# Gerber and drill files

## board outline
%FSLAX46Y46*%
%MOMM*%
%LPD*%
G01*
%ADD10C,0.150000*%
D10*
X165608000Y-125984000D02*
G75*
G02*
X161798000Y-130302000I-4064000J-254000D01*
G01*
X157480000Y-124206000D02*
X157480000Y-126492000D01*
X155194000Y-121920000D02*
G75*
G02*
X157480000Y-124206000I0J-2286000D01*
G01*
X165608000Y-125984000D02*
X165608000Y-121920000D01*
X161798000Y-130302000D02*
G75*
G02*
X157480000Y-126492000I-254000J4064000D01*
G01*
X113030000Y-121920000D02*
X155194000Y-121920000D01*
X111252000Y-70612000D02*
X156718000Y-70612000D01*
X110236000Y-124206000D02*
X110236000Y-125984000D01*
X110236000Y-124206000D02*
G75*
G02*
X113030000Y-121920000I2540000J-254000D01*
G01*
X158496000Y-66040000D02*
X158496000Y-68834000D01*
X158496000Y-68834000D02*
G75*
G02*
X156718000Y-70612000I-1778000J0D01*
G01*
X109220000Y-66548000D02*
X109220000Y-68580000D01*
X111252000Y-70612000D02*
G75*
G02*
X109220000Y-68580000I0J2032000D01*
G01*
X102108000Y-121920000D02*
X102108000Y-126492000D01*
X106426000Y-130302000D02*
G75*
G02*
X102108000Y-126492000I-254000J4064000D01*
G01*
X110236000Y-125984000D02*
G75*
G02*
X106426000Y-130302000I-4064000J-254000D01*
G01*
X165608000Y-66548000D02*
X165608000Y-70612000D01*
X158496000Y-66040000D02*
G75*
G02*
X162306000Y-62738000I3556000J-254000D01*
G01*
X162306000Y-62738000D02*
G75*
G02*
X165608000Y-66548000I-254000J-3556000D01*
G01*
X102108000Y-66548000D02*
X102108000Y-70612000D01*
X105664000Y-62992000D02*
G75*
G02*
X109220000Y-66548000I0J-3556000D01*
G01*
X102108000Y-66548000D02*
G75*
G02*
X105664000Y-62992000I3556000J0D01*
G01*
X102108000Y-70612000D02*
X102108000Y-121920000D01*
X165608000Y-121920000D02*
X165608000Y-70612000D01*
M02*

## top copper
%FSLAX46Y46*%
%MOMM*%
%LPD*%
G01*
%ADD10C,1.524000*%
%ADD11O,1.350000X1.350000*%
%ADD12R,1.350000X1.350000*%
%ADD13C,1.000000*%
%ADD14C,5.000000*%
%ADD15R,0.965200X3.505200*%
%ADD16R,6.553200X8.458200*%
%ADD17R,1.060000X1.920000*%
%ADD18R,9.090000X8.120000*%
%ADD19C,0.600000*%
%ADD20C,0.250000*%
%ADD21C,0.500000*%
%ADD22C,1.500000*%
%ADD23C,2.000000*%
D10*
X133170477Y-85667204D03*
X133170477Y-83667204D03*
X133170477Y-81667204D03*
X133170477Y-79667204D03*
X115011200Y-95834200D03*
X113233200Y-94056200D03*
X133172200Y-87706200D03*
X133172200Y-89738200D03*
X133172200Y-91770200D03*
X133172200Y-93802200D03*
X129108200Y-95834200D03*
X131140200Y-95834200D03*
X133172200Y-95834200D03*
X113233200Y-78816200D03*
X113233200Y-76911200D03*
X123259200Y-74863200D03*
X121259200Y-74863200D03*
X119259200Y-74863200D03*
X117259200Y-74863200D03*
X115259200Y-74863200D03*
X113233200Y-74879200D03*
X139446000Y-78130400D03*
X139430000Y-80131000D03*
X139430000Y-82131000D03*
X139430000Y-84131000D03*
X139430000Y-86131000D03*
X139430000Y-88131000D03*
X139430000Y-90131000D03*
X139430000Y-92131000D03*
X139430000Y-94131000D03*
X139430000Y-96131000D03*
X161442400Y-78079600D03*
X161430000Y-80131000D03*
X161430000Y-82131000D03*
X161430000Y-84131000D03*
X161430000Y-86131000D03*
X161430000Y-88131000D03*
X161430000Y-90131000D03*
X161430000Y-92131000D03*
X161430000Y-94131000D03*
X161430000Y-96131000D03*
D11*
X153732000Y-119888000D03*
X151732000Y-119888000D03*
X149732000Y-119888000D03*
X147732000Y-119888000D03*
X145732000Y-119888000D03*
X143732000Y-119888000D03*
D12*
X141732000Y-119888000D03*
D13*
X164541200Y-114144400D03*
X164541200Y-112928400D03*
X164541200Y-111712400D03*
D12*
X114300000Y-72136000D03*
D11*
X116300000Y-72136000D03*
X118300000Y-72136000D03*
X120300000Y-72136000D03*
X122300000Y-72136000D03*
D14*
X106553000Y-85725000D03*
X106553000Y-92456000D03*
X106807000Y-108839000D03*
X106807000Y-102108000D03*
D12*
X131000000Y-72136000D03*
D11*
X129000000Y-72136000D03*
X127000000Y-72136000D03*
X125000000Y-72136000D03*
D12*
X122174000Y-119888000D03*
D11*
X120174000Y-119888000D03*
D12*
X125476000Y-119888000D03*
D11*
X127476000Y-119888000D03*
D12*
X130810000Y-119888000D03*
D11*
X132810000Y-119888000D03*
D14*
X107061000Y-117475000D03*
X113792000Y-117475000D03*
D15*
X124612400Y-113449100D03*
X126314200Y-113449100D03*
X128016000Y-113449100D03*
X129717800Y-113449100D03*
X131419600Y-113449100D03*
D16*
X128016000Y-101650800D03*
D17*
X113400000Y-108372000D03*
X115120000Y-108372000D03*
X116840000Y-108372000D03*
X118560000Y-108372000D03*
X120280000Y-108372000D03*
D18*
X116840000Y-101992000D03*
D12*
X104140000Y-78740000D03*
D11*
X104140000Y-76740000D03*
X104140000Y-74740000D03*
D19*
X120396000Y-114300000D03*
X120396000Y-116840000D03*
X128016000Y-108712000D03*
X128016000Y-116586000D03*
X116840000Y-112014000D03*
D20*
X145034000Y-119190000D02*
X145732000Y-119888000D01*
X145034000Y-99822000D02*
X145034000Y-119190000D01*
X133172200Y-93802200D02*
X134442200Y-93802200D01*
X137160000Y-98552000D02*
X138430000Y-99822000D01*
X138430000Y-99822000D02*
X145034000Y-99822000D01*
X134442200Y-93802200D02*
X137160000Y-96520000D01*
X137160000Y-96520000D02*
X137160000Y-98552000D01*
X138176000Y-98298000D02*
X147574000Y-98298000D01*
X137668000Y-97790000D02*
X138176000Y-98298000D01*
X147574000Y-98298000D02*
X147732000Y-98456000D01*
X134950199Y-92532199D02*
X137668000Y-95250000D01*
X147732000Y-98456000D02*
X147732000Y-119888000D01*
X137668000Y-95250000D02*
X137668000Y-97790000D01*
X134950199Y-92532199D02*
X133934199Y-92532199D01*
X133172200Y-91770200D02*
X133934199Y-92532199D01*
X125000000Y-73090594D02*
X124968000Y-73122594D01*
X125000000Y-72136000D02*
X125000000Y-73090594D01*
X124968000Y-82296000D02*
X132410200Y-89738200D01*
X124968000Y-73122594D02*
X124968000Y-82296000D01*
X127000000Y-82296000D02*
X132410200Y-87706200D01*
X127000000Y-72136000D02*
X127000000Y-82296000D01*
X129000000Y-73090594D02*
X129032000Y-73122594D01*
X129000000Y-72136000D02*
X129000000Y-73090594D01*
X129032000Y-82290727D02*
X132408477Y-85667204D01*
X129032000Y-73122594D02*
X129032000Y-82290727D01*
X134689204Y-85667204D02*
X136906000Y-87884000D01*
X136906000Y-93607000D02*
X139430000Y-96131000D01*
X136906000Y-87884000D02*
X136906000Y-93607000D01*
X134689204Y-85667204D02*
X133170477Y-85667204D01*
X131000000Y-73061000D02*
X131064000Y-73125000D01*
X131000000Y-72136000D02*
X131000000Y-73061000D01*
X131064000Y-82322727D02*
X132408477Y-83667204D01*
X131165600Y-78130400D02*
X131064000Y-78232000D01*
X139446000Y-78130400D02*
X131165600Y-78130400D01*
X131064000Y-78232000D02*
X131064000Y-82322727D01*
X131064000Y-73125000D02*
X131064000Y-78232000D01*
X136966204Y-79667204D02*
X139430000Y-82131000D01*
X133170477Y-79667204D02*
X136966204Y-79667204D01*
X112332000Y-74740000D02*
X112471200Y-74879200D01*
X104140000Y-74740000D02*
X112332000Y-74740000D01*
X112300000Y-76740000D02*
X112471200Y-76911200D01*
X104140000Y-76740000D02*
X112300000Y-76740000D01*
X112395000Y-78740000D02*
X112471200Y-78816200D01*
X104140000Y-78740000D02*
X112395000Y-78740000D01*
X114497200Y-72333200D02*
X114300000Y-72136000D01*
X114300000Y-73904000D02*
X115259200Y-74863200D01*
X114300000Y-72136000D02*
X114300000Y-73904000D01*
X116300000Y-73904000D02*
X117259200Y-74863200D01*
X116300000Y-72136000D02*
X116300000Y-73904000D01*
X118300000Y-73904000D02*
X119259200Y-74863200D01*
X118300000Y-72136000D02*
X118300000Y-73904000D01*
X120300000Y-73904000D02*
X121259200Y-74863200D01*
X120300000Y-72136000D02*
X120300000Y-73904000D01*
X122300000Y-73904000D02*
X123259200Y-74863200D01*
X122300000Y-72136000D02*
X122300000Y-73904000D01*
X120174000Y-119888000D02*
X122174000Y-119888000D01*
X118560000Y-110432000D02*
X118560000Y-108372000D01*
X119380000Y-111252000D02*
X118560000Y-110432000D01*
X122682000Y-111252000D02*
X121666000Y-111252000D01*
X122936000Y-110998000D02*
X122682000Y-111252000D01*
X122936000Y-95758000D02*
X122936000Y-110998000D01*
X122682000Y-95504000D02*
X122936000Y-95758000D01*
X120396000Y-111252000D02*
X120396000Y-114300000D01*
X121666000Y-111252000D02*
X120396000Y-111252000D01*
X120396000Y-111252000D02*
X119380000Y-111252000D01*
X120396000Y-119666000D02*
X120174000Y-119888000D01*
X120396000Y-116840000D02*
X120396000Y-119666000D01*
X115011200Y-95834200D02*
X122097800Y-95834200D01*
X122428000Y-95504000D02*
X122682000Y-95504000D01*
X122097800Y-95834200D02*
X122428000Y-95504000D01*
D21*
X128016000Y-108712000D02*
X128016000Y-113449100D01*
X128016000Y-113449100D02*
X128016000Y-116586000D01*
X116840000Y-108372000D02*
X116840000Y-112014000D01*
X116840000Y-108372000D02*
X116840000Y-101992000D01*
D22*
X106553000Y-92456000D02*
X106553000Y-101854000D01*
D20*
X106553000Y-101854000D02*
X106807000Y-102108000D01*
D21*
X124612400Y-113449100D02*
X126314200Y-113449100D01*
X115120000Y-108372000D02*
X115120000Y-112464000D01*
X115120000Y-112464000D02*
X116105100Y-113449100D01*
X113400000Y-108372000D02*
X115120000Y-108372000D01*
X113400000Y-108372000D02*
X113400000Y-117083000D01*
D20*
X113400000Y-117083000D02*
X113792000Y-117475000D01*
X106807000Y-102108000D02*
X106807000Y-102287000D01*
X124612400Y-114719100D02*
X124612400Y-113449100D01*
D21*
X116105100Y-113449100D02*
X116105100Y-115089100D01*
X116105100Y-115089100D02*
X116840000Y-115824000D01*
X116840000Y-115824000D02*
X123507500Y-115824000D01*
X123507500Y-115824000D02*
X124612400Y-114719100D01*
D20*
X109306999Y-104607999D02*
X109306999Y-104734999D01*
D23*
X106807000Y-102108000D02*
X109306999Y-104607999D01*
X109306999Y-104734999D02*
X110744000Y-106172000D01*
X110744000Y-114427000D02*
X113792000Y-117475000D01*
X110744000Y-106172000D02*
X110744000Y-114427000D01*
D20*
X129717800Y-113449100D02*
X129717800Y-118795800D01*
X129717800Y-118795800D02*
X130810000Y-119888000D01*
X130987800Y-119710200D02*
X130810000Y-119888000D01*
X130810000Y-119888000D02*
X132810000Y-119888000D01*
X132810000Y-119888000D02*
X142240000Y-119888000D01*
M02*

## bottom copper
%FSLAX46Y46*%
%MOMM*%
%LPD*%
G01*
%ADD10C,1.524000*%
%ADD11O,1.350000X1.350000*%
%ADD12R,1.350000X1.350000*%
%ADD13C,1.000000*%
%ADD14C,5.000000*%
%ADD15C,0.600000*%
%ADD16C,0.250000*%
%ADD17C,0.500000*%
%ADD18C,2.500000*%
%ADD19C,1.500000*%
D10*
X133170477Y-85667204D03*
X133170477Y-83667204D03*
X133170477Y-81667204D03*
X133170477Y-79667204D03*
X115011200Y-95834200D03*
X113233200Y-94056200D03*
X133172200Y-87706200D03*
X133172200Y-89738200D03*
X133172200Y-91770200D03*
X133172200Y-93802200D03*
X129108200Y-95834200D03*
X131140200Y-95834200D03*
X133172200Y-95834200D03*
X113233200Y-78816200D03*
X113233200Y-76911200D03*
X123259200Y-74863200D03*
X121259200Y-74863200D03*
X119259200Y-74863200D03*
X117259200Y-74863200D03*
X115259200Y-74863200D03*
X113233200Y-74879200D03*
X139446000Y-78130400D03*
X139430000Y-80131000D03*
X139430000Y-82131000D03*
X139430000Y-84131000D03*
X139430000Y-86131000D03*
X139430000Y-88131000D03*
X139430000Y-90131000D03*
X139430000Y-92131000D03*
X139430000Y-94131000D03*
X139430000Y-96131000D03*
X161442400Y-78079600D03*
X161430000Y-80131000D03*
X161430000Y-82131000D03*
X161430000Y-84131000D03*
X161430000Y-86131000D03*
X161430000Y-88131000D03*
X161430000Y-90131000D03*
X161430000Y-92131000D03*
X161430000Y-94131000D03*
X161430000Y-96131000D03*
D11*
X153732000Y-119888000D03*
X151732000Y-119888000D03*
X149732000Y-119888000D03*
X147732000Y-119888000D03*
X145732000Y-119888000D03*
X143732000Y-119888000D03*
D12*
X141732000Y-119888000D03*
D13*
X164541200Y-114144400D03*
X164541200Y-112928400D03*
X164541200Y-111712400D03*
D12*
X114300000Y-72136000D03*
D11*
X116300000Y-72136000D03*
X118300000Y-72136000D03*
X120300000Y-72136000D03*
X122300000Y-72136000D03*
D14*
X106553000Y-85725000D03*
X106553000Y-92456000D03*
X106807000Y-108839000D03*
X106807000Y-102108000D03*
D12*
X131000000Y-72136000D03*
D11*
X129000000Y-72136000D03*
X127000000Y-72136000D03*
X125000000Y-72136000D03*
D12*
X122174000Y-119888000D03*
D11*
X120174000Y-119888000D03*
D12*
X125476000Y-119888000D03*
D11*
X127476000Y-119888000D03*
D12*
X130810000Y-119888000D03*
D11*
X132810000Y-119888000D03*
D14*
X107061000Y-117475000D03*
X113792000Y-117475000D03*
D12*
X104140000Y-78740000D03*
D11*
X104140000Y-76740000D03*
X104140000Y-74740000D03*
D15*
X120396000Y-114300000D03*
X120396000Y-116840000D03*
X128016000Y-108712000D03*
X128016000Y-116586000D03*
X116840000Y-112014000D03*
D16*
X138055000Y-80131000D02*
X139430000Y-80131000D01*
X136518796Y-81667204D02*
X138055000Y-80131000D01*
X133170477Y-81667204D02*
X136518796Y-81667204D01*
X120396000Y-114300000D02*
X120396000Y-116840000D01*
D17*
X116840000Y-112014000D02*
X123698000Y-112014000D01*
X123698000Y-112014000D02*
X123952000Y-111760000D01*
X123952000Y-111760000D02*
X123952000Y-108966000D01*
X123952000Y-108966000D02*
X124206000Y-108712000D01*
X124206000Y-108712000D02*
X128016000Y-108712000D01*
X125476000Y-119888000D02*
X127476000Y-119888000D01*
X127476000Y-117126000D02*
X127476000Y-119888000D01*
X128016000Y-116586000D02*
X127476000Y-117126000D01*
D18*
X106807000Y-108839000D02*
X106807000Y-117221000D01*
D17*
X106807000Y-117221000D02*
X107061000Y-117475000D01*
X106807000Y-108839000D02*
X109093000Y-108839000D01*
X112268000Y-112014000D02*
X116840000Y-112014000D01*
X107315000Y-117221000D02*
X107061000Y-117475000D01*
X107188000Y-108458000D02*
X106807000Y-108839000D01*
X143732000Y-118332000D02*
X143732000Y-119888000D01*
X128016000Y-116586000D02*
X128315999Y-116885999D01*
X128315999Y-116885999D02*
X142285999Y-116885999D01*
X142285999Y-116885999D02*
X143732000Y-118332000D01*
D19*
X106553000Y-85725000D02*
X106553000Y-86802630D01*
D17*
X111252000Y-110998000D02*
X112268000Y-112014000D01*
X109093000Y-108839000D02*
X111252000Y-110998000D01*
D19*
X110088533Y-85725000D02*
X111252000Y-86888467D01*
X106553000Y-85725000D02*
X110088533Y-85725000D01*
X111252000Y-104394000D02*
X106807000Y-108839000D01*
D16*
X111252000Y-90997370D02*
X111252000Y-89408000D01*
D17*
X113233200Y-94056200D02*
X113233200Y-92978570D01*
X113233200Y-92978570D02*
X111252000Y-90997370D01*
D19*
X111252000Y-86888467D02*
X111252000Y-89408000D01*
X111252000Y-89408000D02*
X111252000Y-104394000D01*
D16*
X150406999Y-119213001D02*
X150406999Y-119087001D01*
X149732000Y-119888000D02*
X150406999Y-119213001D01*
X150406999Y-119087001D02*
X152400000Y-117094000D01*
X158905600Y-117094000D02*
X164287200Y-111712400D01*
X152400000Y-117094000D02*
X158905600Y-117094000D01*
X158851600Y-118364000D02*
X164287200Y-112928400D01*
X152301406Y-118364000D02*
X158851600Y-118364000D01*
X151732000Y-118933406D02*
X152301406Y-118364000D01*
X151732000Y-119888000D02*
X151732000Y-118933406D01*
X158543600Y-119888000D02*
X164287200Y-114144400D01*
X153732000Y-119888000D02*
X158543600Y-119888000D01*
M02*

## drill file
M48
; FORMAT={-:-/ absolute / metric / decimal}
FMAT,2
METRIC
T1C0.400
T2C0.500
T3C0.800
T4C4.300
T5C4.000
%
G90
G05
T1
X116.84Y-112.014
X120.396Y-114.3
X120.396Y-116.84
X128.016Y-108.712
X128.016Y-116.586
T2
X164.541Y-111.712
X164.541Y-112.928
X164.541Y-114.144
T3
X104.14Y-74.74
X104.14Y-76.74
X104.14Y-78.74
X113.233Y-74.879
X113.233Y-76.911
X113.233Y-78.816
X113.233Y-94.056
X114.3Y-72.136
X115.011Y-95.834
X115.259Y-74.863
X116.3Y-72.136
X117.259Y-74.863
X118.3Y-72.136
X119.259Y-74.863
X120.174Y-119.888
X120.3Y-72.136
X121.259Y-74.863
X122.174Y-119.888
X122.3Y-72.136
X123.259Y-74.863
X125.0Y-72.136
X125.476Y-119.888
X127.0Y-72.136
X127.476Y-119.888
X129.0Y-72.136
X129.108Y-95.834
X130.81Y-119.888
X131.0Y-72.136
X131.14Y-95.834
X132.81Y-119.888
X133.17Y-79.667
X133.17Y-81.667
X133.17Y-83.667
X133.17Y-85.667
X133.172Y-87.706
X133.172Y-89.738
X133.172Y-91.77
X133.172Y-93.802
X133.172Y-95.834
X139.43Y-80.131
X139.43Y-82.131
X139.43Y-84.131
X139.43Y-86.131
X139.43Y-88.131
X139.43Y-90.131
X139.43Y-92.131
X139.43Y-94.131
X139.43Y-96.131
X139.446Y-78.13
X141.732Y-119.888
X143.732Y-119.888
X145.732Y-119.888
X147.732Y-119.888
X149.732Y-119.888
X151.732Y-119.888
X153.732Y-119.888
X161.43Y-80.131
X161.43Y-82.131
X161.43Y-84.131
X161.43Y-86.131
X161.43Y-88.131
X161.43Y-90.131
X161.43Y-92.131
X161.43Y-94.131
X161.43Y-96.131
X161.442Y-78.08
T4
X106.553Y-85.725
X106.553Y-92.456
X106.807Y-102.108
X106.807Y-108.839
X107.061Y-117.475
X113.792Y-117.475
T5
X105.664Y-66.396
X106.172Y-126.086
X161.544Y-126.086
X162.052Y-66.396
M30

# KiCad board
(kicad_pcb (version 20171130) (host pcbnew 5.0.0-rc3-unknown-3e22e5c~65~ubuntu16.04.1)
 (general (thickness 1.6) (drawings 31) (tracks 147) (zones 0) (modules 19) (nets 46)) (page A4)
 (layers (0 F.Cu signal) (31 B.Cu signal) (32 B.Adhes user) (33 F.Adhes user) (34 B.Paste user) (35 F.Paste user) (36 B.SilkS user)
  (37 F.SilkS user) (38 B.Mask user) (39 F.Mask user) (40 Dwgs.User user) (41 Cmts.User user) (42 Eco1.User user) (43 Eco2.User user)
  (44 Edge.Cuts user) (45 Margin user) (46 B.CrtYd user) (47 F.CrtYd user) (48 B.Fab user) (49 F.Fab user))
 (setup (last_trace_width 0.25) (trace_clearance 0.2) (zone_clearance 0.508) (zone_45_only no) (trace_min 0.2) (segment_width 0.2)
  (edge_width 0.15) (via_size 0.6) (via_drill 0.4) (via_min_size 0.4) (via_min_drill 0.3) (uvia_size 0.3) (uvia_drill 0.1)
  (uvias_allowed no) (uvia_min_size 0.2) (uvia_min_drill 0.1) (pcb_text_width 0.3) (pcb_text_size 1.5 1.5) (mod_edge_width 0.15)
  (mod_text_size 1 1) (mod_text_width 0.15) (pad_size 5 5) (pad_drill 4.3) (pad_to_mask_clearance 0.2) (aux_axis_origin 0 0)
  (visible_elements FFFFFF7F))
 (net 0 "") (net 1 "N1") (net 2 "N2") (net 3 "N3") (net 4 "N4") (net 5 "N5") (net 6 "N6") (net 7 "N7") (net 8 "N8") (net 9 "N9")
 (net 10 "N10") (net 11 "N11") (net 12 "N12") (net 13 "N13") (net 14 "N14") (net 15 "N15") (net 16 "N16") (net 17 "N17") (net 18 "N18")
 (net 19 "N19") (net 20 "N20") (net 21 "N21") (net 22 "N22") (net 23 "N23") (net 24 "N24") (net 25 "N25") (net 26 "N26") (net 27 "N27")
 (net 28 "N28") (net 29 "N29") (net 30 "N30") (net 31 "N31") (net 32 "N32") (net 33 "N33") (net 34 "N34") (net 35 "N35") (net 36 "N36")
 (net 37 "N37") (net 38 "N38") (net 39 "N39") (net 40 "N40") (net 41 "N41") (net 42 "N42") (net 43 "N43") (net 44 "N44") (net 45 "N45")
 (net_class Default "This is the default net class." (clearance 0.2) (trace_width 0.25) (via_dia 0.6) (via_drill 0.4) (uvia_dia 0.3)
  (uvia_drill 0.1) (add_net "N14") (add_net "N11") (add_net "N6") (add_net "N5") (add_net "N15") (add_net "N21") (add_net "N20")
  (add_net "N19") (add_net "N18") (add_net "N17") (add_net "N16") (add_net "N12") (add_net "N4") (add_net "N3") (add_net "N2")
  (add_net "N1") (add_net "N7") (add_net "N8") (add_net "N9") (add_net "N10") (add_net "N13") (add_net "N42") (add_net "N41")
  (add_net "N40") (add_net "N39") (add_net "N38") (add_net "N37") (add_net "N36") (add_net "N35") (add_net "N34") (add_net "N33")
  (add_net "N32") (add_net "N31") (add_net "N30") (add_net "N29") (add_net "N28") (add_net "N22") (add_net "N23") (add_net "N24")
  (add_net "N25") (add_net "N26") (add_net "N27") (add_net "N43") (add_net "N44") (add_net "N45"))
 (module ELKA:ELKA (layer F.Cu) (at 122.428 85.852)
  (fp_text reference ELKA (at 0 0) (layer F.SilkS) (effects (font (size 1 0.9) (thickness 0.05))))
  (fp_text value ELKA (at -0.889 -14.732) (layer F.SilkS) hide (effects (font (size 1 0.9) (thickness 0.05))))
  (pad D thru_hole circle (at 10.742477 -0.184796 270) (size 1.524 1.524) (drill 0.8) (layers *.Cu *.Mask B.SilkS) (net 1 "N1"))
  (pad C thru_hole circle (at 10.742477 -2.184796 270) (size 1.524 1.524) (drill 0.8) (layers *.Cu *.Mask B.SilkS) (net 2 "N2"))
  (pad B thru_hole circle (at 10.742477 -4.184796 270) (size 1.524 1.524) (drill 0.8) (layers *.Cu *.Mask B.SilkS) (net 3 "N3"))
  (pad A thru_hole circle (at 10.742477 -6.184796 270) (size 1.524 1.524) (drill 0.8) (layers *.Cu *.Mask B.SilkS) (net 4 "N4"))
  (pad 12 thru_hole circle (at -7.4168 9.9822 270) (size 1.524 1.524) (drill 0.8) (layers *.Cu *.Mask B.SilkS) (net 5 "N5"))
  (pad 11 thru_hole circle (at -9.1948 8.2042 270) (size 1.524 1.524) (drill 0.8) (layers *.Cu *.Mask B.SilkS) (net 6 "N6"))
  (pad E thru_hole circle (at 10.7442 1.8542 270) (size 1.524 1.524) (drill 0.8) (layers *.Cu *.Mask B.SilkS) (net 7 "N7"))
  (pad F thru_hole circle (at 10.7442 3.8862 270) (size 1.524 1.524) (drill 0.8) (layers *.Cu *.Mask B.SilkS) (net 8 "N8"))
  (pad G thru_hole circle (at 10.7442 5.9182 270) (size 1.524 1.524) (drill 0.8) (layers *.Cu *.Mask B.SilkS) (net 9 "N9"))
  (pad H thru_hole circle (at 10.7442 7.9502 270) (size 1.524 1.524) (drill 0.8) (layers *.Cu *.Mask B.SilkS) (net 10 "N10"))
  (pad 10 thru_hole circle (at 6.6802 9.9822 270) (size 1.524 1.524) (drill 0.8) (layers *.Cu *.Mask B.SilkS) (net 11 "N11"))
  (pad 9 thru_hole circle (at 8.7122 9.9822 270) (size 1.524 1.524) (drill 0.8) (layers *.Cu *.Mask B.SilkS) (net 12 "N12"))
  (pad I thru_hole circle (at 10.7442 9.9822 270) (size 1.524 1.524) (drill 0.8) (layers *.Cu *.Mask B.SilkS) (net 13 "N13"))
  (pad 1 thru_hole circle (at -9.1948 -7.0358 270) (size 1.524 1.524) (drill 0.8) (layers *.Cu *.Mask B.SilkS) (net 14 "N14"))
  (pad 2 thru_hole circle (at -9.1948 -8.9408 270) (size 1.524 1.524) (drill 0.8) (layers *.Cu *.Mask B.SilkS) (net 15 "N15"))
  (pad 8 thru_hole circle (at 0.8312 -10.9888 270) (size 1.524 1.524) (drill 0.8) (layers *.Cu *.Mask B.SilkS) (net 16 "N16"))
  (pad 7 thru_hole circle (at -1.1688 -10.9888 270) (size 1.524 1.524) (drill 0.8) (layers *.Cu *.Mask B.SilkS) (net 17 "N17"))
  (pad 6 thru_hole circle (at -3.1688 -10.9888 270) (size 1.524 1.524) (drill 0.8) (layers *.Cu *.Mask B.SilkS) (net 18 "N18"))
  (pad 5 thru_hole circle (at -5.1688 -10.9888 270) (size 1.524 1.524) (drill 0.8) (layers *.Cu *.Mask B.SilkS) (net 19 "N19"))
  (pad 4 thru_hole circle (at -7.1688 -10.9888 270) (size 1.524 1.524) (drill 0.8) (layers *.Cu *.Mask B.SilkS) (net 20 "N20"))
  (pad 3 thru_hole circle (at -9.1948 -10.9728 270) (size 1.524 1.524) (drill 0.8) (layers *.Cu *.Mask B.SilkS) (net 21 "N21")))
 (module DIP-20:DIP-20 (layer F.Cu) (at 138.176 104.14)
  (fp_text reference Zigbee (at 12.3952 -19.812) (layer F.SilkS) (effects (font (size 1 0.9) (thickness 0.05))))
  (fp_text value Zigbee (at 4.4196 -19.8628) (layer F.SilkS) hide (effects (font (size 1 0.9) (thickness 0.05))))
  (pad 1 thru_hole circle (at 1.27 -26.0096) (size 1.524 1.524) (drill 0.8) (layers *.Cu *.Mask F.SilkS) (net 2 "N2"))
  (pad 2 thru_hole circle (at 1.254 -24.009) (size 1.524 1.524) (drill 0.8) (layers *.Cu *.Mask F.SilkS) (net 3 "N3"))
  (pad 3 thru_hole circle (at 1.254 -22.009) (size 1.524 1.524) (drill 0.8) (layers *.Cu *.Mask F.SilkS) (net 4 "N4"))
  (pad 4 thru_hole circle (at 1.254 -20.009) (size 1.524 1.524) (drill 0.8) (layers *.Cu *.Mask F.SilkS) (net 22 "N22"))
  (pad 5 thru_hole circle (at 1.254 -18.009) (size 1.524 1.524) (drill 0.8) (layers *.Cu *.Mask F.SilkS) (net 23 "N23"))
  (pad 6 thru_hole circle (at 1.254 -16.009) (size 1.524 1.524) (drill 0.8) (layers *.Cu *.Mask F.SilkS) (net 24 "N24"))
  (pad 7 thru_hole circle (at 1.254 -14.009) (size 1.524 1.524) (drill 0.8) (layers *.Cu *.Mask F.SilkS) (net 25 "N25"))
  (pad 8 thru_hole circle (at 1.254 -12.009) (size 1.524 1.524) (drill 0.8) (layers *.Cu *.Mask F.SilkS) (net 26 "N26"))
  (pad 9 thru_hole circle (at 1.254 -10.009) (size 1.524 1.524) (drill 0.8) (layers *.Cu *.Mask F.SilkS) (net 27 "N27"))
  (pad 10 thru_hole circle (at 1.254 -8.009) (size 1.524 1.524) (drill 0.8) (layers *.Cu *.Mask F.SilkS) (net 1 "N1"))
  (pad 20 thru_hole circle (at 23.2664 -26.0604) (size 1.524 1.524) (drill 0.8) (layers *.Cu *.Mask F.SilkS) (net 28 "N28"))
  (pad 19 thru_hole circle (at 23.254 -24.009) (size 1.524 1.524) (drill 0.8) (layers *.Cu *.Mask F.SilkS) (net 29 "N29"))
  (pad 18 thru_hole circle (at 23.254 -22.009) (size 1.524 1.524) (drill 0.8) (layers *.Cu *.Mask F.SilkS) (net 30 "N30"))
  (pad 17 thru_hole circle (at 23.254 -20.009) (size 1.524 1.524) (drill 0.8) (layers *.Cu *.Mask F.SilkS) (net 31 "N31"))
  (pad 16 thru_hole circle (at 23.254 -18.009) (size 1.524 1.524) (drill 0.8) (layers *.Cu *.Mask F.SilkS) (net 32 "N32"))
  (pad 15 thru_hole circle (at 23.254 -16.009) (size 1.524 1.524) (drill 0.8) (layers *.Cu *.Mask F.SilkS) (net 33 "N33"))
  (pad 14 thru_hole circle (at 23.254 -14.009) (size 1.524 1.524) (drill 0.8) (layers *.Cu *.Mask F.SilkS) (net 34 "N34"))
  (pad 13 thru_hole circle (at 23.254 -12.009) (size 1.524 1.524) (drill 0.8) (layers *.Cu *.Mask F.SilkS) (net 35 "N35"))
  (pad 12 thru_hole circle (at 23.254 -10.009) (size 1.524 1.524) (drill 0.8) (layers *.Cu *.Mask F.SilkS) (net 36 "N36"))
  (pad 11 thru_hole circle (at 23.254 -8.009) (size 1.524 1.524) (drill 0.8) (layers *.Cu *.Mask F.SilkS) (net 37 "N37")))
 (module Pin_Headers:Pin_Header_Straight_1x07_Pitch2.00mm (layer F.Cu) (at 141.732 119.888 90)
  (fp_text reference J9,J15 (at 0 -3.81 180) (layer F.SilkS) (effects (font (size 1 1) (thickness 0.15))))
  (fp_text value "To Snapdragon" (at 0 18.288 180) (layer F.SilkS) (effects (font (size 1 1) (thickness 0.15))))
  (pad 5 thru_hole oval (at 0 12 90) (size 1.35 1.35) (drill 0.8) (layers *.Cu *.Mask) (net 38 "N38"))
  (pad 4 thru_hole oval (at 0 10 90) (size 1.35 1.35) (drill 0.8) (layers *.Cu *.Mask) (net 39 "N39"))
  (pad 3 thru_hole oval (at 0 8 90) (size 1.35 1.35) (drill 0.8) (layers *.Cu *.Mask) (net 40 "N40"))
  (pad 6 thru_hole oval (at 0 6 90) (size 1.35 1.35) (drill 0.8) (layers *.Cu *.Mask) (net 9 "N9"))
  (pad 7 thru_hole oval (at 0 4 90) (size 1.35 1.35) (drill 0.8) (layers *.Cu *.Mask) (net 10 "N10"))
  (pad 2 thru_hole oval (at 0 2 90) (size 1.35 1.35) (drill 0.8) (layers *.Cu *.Mask) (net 6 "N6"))
  (pad 1 thru_hole rect (at 0 0 90) (size 1.35 1.35) (drill 0.8) (layers *.Cu *.Mask) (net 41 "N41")))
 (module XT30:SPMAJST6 (layer F.Cu) (at 163.83 113.792 270)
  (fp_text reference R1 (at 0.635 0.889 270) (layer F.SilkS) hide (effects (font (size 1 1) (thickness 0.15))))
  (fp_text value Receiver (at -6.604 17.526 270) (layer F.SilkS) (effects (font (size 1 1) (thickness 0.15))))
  (pad 3 thru_hole circle (at 0.3524 -0.7112 270) (size 1 1) (drill 0.5) (layers *.Cu *.Mask) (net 38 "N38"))
  (pad 2 thru_hole circle (at -0.8636 -0.7112 270) (size 1 1) (drill 0.5) (layers *.Cu *.Mask) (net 39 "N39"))
  (pad 1 thru_hole circle (at -2.0796 -0.7112 270) (size 1 1) (drill 0.5) (layers *.Cu *.Mask) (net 40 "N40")))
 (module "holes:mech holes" (layer F.Cu) (at 162.052 129.286)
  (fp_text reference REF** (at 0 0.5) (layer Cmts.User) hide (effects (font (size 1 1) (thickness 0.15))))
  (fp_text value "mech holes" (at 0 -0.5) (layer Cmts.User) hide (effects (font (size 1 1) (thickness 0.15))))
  (pad "" np_thru_hole circle (at -0.508 -3.2004) (size 4 4) (drill 4) (layers *.Cu *.Mask)))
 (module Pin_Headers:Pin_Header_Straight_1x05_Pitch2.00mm (layer F.Cu) (at 114.3 72.136 90)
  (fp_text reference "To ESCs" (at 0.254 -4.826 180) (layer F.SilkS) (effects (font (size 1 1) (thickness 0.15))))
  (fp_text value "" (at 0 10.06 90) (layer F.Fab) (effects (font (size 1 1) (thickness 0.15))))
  (pad 1 thru_hole rect (at 0 0 90) (size 1.35 1.35) (drill 0.8) (layers *.Cu *.Mask) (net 20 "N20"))
  (pad 2 thru_hole oval (at 0 2 90) (size 1.35 1.35) (drill 0.8) (layers *.Cu *.Mask) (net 19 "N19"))
  (pad 3 thru_hole oval (at 0 4 90) (size 1.35 1.35) (drill 0.8) (layers *.Cu *.Mask) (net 18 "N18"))
  (pad 4 thru_hole oval (at 0 6 90) (size 1.35 1.35) (drill 0.8) (layers *.Cu *.Mask) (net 17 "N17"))
  (pad 5 thru_hole oval (at 0 8 90) (size 1.35 1.35) (drill 0.8) (layers *.Cu *.Mask) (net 16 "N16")))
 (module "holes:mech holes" (layer F.Cu) (at 106.172 69.596)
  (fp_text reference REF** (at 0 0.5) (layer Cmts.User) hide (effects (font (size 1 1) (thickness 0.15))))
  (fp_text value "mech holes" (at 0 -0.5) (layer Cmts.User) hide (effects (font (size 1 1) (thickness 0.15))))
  (pad "" np_thru_hole circle (at -0.508 -3.2004) (size 4 4) (drill 4) (layers *.Cu *.Mask)))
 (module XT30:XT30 (layer F.Cu) (at 112.522 87.122 270)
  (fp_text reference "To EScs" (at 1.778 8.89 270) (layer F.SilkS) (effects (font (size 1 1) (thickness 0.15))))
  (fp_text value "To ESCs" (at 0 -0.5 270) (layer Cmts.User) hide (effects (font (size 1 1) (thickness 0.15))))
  (pad 1 thru_hole circle (at -1.397 5.969 270) (size 5 5) (drill 4.3) (layers *.Cu *.Mask) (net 6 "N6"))
  (pad 2 thru_hole circle (at 5.334 5.969 270) (size 5 5) (drill 4.3) (layers *.Cu *.Mask) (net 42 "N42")))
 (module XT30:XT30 (layer F.Cu) (at 100.838 107.442 90)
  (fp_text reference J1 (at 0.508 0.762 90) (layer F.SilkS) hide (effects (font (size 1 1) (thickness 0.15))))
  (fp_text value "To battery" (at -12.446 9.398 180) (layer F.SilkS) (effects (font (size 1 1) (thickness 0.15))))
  (pad 1 thru_hole circle (at -1.397 5.969 90) (size 5 5) (drill 4.3) (layers *.Cu *.Mask) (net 6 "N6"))
  (pad 2 thru_hole circle (at 5.334 5.969 90) (size 5 5) (drill 4.3) (layers *.Cu *.Mask) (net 42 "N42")))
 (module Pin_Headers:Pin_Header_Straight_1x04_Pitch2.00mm (layer F.Cu) (at 131 72.136 270)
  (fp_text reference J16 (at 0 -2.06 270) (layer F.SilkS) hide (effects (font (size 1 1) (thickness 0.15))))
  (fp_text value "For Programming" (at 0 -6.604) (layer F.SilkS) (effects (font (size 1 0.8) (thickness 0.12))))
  (pad 1 thru_hole rect (at 0 0 270) (size 1.35 1.35) (drill 0.8) (layers *.Cu *.Mask) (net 2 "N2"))
  (pad 2 thru_hole oval (at 0 2 270) (size 1.35 1.35) (drill 0.8) (layers *.Cu *.Mask) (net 1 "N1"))
  (pad 3 thru_hole oval (at 0 4 270) (size 1.35 1.35) (drill 0.8) (layers *.Cu *.Mask) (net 7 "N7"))
  (pad 4 thru_hole oval (at 0 6 270) (size 1.35 1.35) (drill 0.8) (layers *.Cu *.Mask) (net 8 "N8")))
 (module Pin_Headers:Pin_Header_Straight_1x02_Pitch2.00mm (layer F.Cu) (at 122.174 119.888 270)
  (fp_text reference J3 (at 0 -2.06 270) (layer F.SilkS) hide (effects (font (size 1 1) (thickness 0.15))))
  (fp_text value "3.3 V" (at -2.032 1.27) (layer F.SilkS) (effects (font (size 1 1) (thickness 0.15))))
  (pad 1 thru_hole rect (at 0 0 270) (size 1.35 1.35) (drill 0.8) (layers *.Cu *.Mask) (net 5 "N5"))
  (pad 2 thru_hole oval (at 0 2 270) (size 1.35 1.35) (drill 0.8) (layers *.Cu *.Mask) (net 5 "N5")))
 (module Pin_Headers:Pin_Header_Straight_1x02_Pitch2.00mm (layer F.Cu) (at 125.476 119.888 90)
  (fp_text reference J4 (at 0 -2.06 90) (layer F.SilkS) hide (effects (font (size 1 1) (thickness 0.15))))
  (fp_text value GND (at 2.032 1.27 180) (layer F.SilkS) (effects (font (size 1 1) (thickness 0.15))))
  (pad 1 thru_hole rect (at 0 0 90) (size 1.35 1.35) (drill 0.8) (layers *.Cu *.Mask) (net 6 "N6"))
  (pad 2 thru_hole oval (at 0 2 90) (size 1.35 1.35) (drill 0.8) (layers *.Cu *.Mask) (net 6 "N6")))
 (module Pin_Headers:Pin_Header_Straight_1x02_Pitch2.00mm (layer F.Cu) (at 130.81 119.888 90)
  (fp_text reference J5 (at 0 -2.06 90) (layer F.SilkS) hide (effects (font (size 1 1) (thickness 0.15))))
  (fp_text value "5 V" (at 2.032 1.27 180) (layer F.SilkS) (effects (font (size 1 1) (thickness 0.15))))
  (pad 1 thru_hole rect (at 0 0 90) (size 1.35 1.35) (drill 0.8) (layers *.Cu *.Mask) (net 41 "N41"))
  (pad 2 thru_hole oval (at 0 2 90) (size 1.35 1.35) (drill 0.8) (layers *.Cu *.Mask) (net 41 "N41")))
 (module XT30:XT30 (layer F.Cu) (at 108.458 111.506)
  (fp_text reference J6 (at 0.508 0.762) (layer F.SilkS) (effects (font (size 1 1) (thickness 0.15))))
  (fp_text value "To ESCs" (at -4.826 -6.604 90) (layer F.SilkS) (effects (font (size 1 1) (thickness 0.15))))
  (pad 1 thru_hole circle (at -1.397 5.969) (size 5 5) (drill 4.3) (layers *.Cu *.Mask) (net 6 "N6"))
  (pad 2 thru_hole circle (at 5.334 5.969) (size 5 5) (drill 4.3) (layers *.Cu *.Mask) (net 42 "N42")))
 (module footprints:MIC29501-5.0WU (layer F.Cu) (at 128.016 104.394)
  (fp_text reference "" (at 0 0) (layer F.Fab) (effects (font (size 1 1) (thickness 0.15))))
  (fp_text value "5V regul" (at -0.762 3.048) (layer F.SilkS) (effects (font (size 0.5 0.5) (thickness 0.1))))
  (pad 1 smd rect (at -3.4036 9.0551) (size 0.9652 3.5052) (layers F.Cu F.Paste F.Mask) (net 42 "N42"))
  (pad 2 smd rect (at -1.7018 9.0551) (size 0.9652 3.5052) (layers F.Cu F.Paste F.Mask) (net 42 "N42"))
  (pad 3 smd rect (at 0 9.0551) (size 0.9652 3.5052) (layers F.Cu F.Paste F.Mask) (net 6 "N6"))
  (pad 4 smd rect (at 1.7018 9.0551) (size 0.9652 3.5052) (layers F.Cu F.Paste F.Mask) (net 41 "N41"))
  (pad 5 smd rect (at 3.4036 9.0551) (size 0.9652 3.5052) (layers F.Cu F.Paste F.Mask) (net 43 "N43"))
  (pad 6 smd rect (at 0 -2.7432) (size 6.5532 8.4582) (layers F.Cu F.Paste F.Mask) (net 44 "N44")))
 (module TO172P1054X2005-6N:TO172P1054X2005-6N (layer F.Cu) (at 116.84 103.632)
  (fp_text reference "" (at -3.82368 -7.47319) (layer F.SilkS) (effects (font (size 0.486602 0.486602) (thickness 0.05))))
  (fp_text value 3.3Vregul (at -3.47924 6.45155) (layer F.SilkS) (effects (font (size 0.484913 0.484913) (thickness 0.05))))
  (pad 1 smd rect (at -3.44 4.74 90) (size 1.92 1.06) (layers F.Cu F.Paste F.Mask) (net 42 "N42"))
  (pad 2 smd rect (at -1.72 4.74 90) (size 1.92 1.06) (layers F.Cu F.Paste F.Mask) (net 42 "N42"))
  (pad 3 smd rect (at 0 4.74 90) (size 1.92 1.06) (layers F.Cu F.Paste F.Mask) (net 6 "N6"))
  (pad 4 smd rect (at 1.72 4.74 90) (size 1.92 1.06) (layers F.Cu F.Paste F.Mask) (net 5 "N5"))
  (pad 5 smd rect (at 3.44 4.74 90) (size 1.92 1.06) (layers F.Cu F.Paste F.Mask) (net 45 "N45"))
  (pad 6 smd rect (at 0 -1.64 90) (size 8.12 9.09) (layers F.Cu F.Paste F.Mask) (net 6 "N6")))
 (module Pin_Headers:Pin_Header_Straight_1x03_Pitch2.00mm (layer F.Cu) (at 104.14 78.74 180)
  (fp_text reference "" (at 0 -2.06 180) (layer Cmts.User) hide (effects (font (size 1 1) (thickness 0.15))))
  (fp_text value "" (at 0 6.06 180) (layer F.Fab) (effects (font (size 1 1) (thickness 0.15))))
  (pad 1 thru_hole rect (at 0 0 180) (size 1.35 1.35) (drill 0.8) (layers *.Cu *.Mask) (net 14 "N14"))
  (pad 2 thru_hole oval (at 0 2 180) (size 1.35 1.35) (drill 0.8) (layers *.Cu *.Mask) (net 15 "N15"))
  (pad 3 thru_hole oval (at 0 4 180) (size 1.35 1.35) (drill 0.8) (layers *.Cu *.Mask) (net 21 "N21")))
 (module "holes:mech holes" (layer F.Cu) (at 162.56 69.596)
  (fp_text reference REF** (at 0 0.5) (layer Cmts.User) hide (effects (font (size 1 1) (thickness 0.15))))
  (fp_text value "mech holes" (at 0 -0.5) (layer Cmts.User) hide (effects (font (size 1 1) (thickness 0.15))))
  (pad "" np_thru_hole circle (at -0.508 -3.2004) (size 4 4) (drill 4) (layers *.Cu *.Mask)))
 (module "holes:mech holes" (layer F.Cu) (at 106.68 129.286)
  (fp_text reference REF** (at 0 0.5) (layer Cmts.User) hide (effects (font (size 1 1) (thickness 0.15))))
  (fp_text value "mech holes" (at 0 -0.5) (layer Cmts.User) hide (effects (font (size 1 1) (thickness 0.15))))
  (pad "" np_thru_hole circle (at -0.508 -3.2004) (size 4 4) (drill 4) (layers *.Cu *.Mask)))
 (gr_arc (start 161.544 126.238) (end 165.608 125.984) (angle 90) (layer Edge.Cuts) (width 0.15))
 (gr_line (start 157.48 124.206) (end 157.48 126.492) (angle 90) (layer Edge.Cuts) (width 0.15))
 (gr_arc (start 155.194 124.206) (end 155.194 121.92) (angle 90) (layer Edge.Cuts) (width 0.15))
 (gr_line (start 165.608 125.984) (end 165.608 121.92) (angle 90) (layer Edge.Cuts) (width 0.15))
 (gr_arc (start 161.544 126.238) (end 161.798 130.302) (angle 90) (layer Edge.Cuts) (width 0.15))
 (gr_line (start 113.03 121.92) (end 155.194 121.92) (angle 90) (layer Edge.Cuts) (width 0.15))
 (gr_line (start 111.252 70.612) (end 156.718 70.612) (angle 90) (layer Edge.Cuts) (width 0.15))
 (gr_line (start 110.236 124.206) (end 110.236 125.984) (angle 90) (layer Edge.Cuts) (width 0.15))
 (gr_arc (start 112.776 124.46) (end 110.236 124.206) (angle 90) (layer Edge.Cuts) (width 0.15))
 (gr_line (start 158.496 66.04) (end 158.496 68.834) (angle 90) (layer Edge.Cuts) (width 0.15))
 (gr_arc (start 156.718 68.834) (end 158.496 68.834) (angle 90) (layer Edge.Cuts) (width 0.15))
 (gr_line (start 109.22 66.548) (end 109.22 68.58) (angle 90) (layer Edge.Cuts) (width 0.15))
 (gr_arc (start 111.252 68.58) (end 111.252 70.612) (angle 90) (layer Edge.Cuts) (width 0.15))
 (gr_line (start 102.108 121.92) (end 102.108 126.492) (angle 90) (layer Edge.Cuts) (width 0.15))
 (gr_arc (start 106.172 126.238) (end 106.426 130.302) (angle 90) (layer Edge.Cuts) (width 0.15))
 (gr_arc (start 106.172 126.238) (end 110.236 125.984) (angle 90) (layer Edge.Cuts) (width 0.15))
 (gr_line (start 165.608 66.548) (end 165.608 70.612) (angle 90) (layer Edge.Cuts) (width 0.15))
 (gr_arc (start 162.052 66.294) (end 158.496 66.04) (angle 90) (layer Edge.Cuts) (width 0.15))
 (gr_arc (start 162.052 66.294) (end 162.306 62.738) (angle 90) (layer Edge.Cuts) (width 0.15))
 (gr_line (start 102.108 66.548) (end 102.108 70.612) (angle 90) (layer Edge.Cuts) (width 0.15))
 (gr_arc (start 105.664 66.548) (end 105.664 62.992) (angle 90) (layer Edge.Cuts) (width 0.15))
 (gr_arc (start 105.664 66.548) (end 102.108 66.548) (angle 90) (layer Edge.Cuts) (width 0.15))
 (gr_line (start 102.108 70.612) (end 102.108 121.92) (angle 90) (layer Edge.Cuts) (width 0.15))
 (gr_line (start 165.608 121.92) (end 165.608 70.612) (angle 90) (layer Edge.Cuts) (width 0.15))
 (segment (start 145.034 119.19) (end 145.732 119.888) (width 0.25) (layer F.Cu) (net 10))
 (segment (start 145.034 99.822) (end 145.034 119.19) (width 0.25) (layer F.Cu) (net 10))
 (segment (start 133.1722 93.8022) (end 134.4422 93.8022) (width 0.25) (layer F.Cu) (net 10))
 (segment (start 137.16 98.552) (end 138.43 99.822) (width 0.25) (layer F.Cu) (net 10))
 (segment (start 138.43 99.822) (end 145.034 99.822) (width 0.25) (layer F.Cu) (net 10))
 (segment (start 134.4422 93.8022) (end 137.16 96.52) (width 0.25) (layer F.Cu) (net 10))
 (segment (start 137.16 96.52) (end 137.16 98.552) (width 0.25) (layer F.Cu) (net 10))
 (segment (start 138.176 98.298) (end 147.574 98.298) (width 0.25) (layer F.Cu) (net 9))
 (segment (start 137.668 97.79) (end 138.176 98.298) (width 0.25) (layer F.Cu) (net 9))
 (segment (start 147.574 98.298) (end 147.732 98.456) (width 0.25) (layer F.Cu) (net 9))
 (segment (start 134.950199 92.532199) (end 137.668 95.25) (width 0.25) (layer F.Cu) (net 9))
 (segment (start 147.732 98.456) (end 147.732 119.888) (width 0.25) (layer F.Cu) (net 9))
 (segment (start 137.668 95.25) (end 137.668 97.79) (width 0.25) (layer F.Cu) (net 9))
 (segment (start 134.950199 92.532199) (end 133.934199 92.532199) (width 0.25) (layer F.Cu) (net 9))
 (segment (start 133.1722 91.7702) (end 133.934199 92.532199) (width 0.25) (layer F.Cu) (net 9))
 (segment (start 125 73.090594) (end 124.968 73.122594) (width 0.25) (layer F.Cu) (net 8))
 (segment (start 125 72.136) (end 125 73.090594) (width 0.25) (layer F.Cu) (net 8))
 (segment (start 124.968 82.296) (end 132.4102 89.7382) (width 0.25) (layer F.Cu) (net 8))
 (segment (start 124.968 73.122594) (end 124.968 82.296) (width 0.25) (layer F.Cu) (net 8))
 (segment (start 127 82.296) (end 132.4102 87.7062) (width 0.25) (layer F.Cu) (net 7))
 (segment (start 127 72.136) (end 127 82.296) (width 0.25) (layer F.Cu) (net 7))
 (segment (start 129 73.090594) (end 129.032 73.122594) (width 0.25) (layer F.Cu) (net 1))
 (segment (start 129 72.136) (end 129 73.090594) (width 0.25) (layer F.Cu) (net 1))
 (segment (start 129.032 82.290727) (end 132.408477 85.667204) (width 0.25) (layer F.Cu) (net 1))
 (segment (start 129.032 73.122594) (end 129.032 82.290727) (width 0.25) (layer F.Cu) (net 1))
 (segment (start 134.689204 85.667204) (end 136.906 87.884) (width 0.25) (layer F.Cu) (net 1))
 (segment (start 136.906 93.607) (end 139.43 96.131) (width 0.25) (layer F.Cu) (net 1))
 (segment (start 136.906 87.884) (end 136.906 93.607) (width 0.25) (layer F.Cu) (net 1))
 (segment (start 134.689204 85.667204) (end 133.170477 85.667204) (width 0.25) (layer F.Cu) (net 1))
 (segment (start 131 73.061) (end 131.064 73.125) (width 0.25) (layer F.Cu) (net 2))
 (segment (start 131 72.136) (end 131 73.061) (width 0.25) (layer F.Cu) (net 2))
 (segment (start 131.064 82.322727) (end 132.408477 83.667204) (width 0.25) (layer F.Cu) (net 2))
 (segment (start 131.1656 78.1304) (end 131.064 78.232) (width 0.25) (layer F.Cu) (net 2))
 (segment (start 139.446 78.1304) (end 131.1656 78.1304) (width 0.25) (layer F.Cu) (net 2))
 (segment (start 131.064 78.232) (end 131.064 82.322727) (width 0.25) (layer F.Cu) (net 2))
 (segment (start 131.064 73.125) (end 131.064 78.232) (width 0.25) (layer F.Cu) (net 2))
 (segment (start 138.055 80.131) (end 139.43 80.131) (width 0.25) (layer B.Cu) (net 3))
 (segment (start 136.518796 81.667204) (end 138.055 80.131) (width 0.25) (layer B.Cu) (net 3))
 (segment (start 133.170477 81.667204) (end 136.518796 81.667204) (width 0.25) (layer B.Cu) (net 3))
 (segment (start 136.966204 79.667204) (end 139.43 82.131) (width 0.25) (layer F.Cu) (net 4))
 (segment (start 133.170477 79.667204) (end 136.966204 79.667204) (width 0.25) (layer F.Cu) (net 4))
 (segment (start 112.332 74.74) (end 112.4712 74.8792) (width 0.25) (layer F.Cu) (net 21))
 (segment (start 104.14 74.74) (end 112.332 74.74) (width 0.25) (layer F.Cu) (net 21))
 (segment (start 112.3 76.74) (end 112.4712 76.9112) (width 0.25) (layer F.Cu) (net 15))
 (segment (start 104.14 76.74) (end 112.3 76.74) (width 0.25) (layer F.Cu) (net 15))
 (segment (start 112.395 78.74) (end 112.4712 78.8162) (width 0.25) (layer F.Cu) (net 14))
 (segment (start 104.14 78.74) (end 112.395 78.74) (width 0.25) (layer F.Cu) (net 14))
 (segment (start 114.4972 72.3332) (end 114.3 72.136) (width 0.25) (layer F.Cu) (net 20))
 (segment (start 114.3 73.904) (end 115.2592 74.8632) (width 0.25) (layer F.Cu) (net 20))
 (segment (start 114.3 72.136) (end 114.3 73.904) (width 0.25) (layer F.Cu) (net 20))
 (segment (start 116.3 73.904) (end 117.2592 74.8632) (width 0.25) (layer F.Cu) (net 19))
 (segment (start 116.3 72.136) (end 116.3 73.904) (width 0.25) (layer F.Cu) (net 19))
 (segment (start 118.3 73.904) (end 119.2592 74.8632) (width 0.25) (layer F.Cu) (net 18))
 (segment (start 118.3 72.136) (end 118.3 73.904) (width 0.25) (layer F.Cu) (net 18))
 (segment (start 120.3 73.904) (end 121.2592 74.8632) (width 0.25) (layer F.Cu) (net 17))
 (segment (start 120.3 72.136) (end 120.3 73.904) (width 0.25) (layer F.Cu) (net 17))
 (segment (start 122.3 73.904) (end 123.2592 74.8632) (width 0.25) (layer F.Cu) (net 16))
 (segment (start 122.3 72.136) (end 122.3 73.904) (width 0.25) (layer F.Cu) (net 16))
 (segment (start 120.174 119.888) (end 122.174 119.888) (width 0.25) (layer F.Cu) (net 5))
 (segment (start 118.56 110.432) (end 118.56 108.372) (width 0.25) (layer F.Cu) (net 5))
 (segment (start 119.38 111.252) (end 118.56 110.432) (width 0.25) (layer F.Cu) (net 5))
 (segment (start 122.682 111.252) (end 121.666 111.252) (width 0.25) (layer F.Cu) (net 5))
 (segment (start 122.936 110.998) (end 122.682 111.252) (width 0.25) (layer F.Cu) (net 5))
 (segment (start 122.936 95.758) (end 122.936 110.998) (width 0.25) (layer F.Cu) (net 5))
 (segment (start 122.682 95.504) (end 122.936 95.758) (width 0.25) (layer F.Cu) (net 5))
 (segment (start 120.396 111.252) (end 120.396 114.3) (width 0.25) (layer F.Cu) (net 5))
 (via (at 120.396 114.3) (size 0.6) (drill 0.4) (layers F.Cu B.Cu) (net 5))
 (segment (start 121.666 111.252) (end 120.396 111.252) (width 0.25) (layer F.Cu) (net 5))
 (segment (start 120.396 111.252) (end 119.38 111.252) (width 0.25) (layer F.Cu) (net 5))
 (via (at 120.396 116.84) (size 0.6) (drill 0.4) (layers F.Cu B.Cu) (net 5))
 (segment (start 120.396 114.3) (end 120.396 116.84) (width 0.25) (layer B.Cu) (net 5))
 (segment (start 120.396 119.666) (end 120.174 119.888) (width 0.25) (layer F.Cu) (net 5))
 (segment (start 120.396 116.84) (end 120.396 119.666) (width 0.25) (layer F.Cu) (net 5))
 (segment (start 115.0112 95.8342) (end 122.0978 95.8342) (width 0.25) (layer F.Cu) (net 5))
 (segment (start 122.428 95.504) (end 122.682 95.504) (width 0.25) (layer F.Cu) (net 5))
 (segment (start 122.0978 95.8342) (end 122.428 95.504) (width 0.25) (layer F.Cu) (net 5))
 (segment (start 116.84 112.014) (end 123.698 112.014) (width 0.5) (layer B.Cu) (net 6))
 (segment (start 123.698 112.014) (end 123.952 111.76) (width 0.5) (layer B.Cu) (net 6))
 (segment (start 123.952 111.76) (end 123.952 108.966) (width 0.5) (layer B.Cu) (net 6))
 (segment (start 123.952 108.966) (end 124.206 108.712) (width 0.5) (layer B.Cu) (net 6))
 (segment (start 124.206 108.712) (end 128.016 108.712) (width 0.5) (layer B.Cu) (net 6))
 (via (at 128.016 108.712) (size 0.6) (drill 0.4) (layers F.Cu B.Cu) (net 6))
 (segment (start 128.016 108.712) (end 128.016 113.4491) (width 0.5) (layer F.Cu) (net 6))
 (segment (start 125.476 119.888) (end 127.476 119.888) (width 0.5) (layer B.Cu) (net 6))
 (segment (start 128.016 113.4491) (end 128.016 116.586) (width 0.5) (layer F.Cu) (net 6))
 (via (at 128.016 116.586) (size 0.6) (drill 0.4) (layers F.Cu B.Cu) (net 6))
 (segment (start 127.476 117.126) (end 127.476 119.888) (width 0.5) (layer B.Cu) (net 6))
 (segment (start 128.016 116.586) (end 127.476 117.126) (width 0.5) (layer B.Cu) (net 6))
 (segment (start 106.807 108.839) (end 106.807 117.221) (width 2.5) (layer B.Cu) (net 6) (status 10))
 (segment (start 106.807 117.221) (end 107.061 117.475) (width 0.5) (layer B.Cu) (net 6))
 (segment (start 116.84 108.372) (end 116.84 112.014) (width 0.5) (layer F.Cu) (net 6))
 (via (at 116.84 112.014) (size 0.6) (drill 0.4) (layers F.Cu B.Cu) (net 6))
 (segment (start 106.807 108.839) (end 109.093 108.839) (width 0.5) (layer B.Cu) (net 6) (status 10))
 (segment (start 112.268 112.014) (end 116.84 112.014) (width 0.5) (layer B.Cu) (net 6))
 (segment (start 107.315 117.221) (end 107.061 117.475) (width 0.5) (layer B.Cu) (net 6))
 (segment (start 107.188 108.458) (end 106.807 108.839) (width 0.5) (layer B.Cu) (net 6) (status 30))
 (segment (start 116.84 108.372) (end 116.84 101.992) (width 0.5) (layer F.Cu) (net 6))
 (segment (start 143.732 118.332) (end 143.732 119.888) (width 0.5) (layer B.Cu) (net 6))
 (segment (start 128.016 116.586) (end 128.315999 116.885999) (width 0.5) (layer B.Cu) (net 6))
 (segment (start 128.315999 116.885999) (end 142.285999 116.885999) (width 0.5) (layer B.Cu) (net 6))
 (segment (start 142.285999 116.885999) (end 143.732 118.332) (width 0.5) (layer B.Cu) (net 6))
 (segment (start 106.553 85.725) (end 106.553 86.80263) (width 1.5) (layer B.Cu) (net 6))
 (segment (start 111.252 110.998) (end 112.268 112.014) (width 0.5) (layer B.Cu) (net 6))
 (segment (start 109.093 108.839) (end 111.252 110.998) (width 0.5) (layer B.Cu) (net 6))
 (segment (start 110.088533 85.725) (end 111.252 86.888467) (width 1.5) (layer B.Cu) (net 6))
 (segment (start 106.553 85.725) (end 110.088533 85.725) (width 1.5) (layer B.Cu) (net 6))
 (segment (start 111.252 104.394) (end 106.807 108.839) (width 1.5) (layer B.Cu) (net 6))
 (segment (start 111.252 90.99737) (end 111.252 89.408) (width 0.25) (layer B.Cu) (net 6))
 (segment (start 113.2332 94.0562) (end 113.2332 92.97857) (width 0.5) (layer B.Cu) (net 6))
 (segment (start 113.2332 92.97857) (end 111.252 90.99737) (width 0.5) (layer B.Cu) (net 6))
 (segment (start 111.252 86.888467) (end 111.252 89.408) (width 1.5) (layer B.Cu) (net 6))
 (segment (start 111.252 89.408) (end 111.252 104.394) (width 1.5) (layer B.Cu) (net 6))
 (segment (start 106.553 92.456) (end 106.553 101.854) (width 1.5) (layer F.Cu) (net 42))
 (segment (start 106.553 101.854) (end 106.807 102.108) (width 0.25) (layer F.Cu) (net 42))
 (segment (start 124.6124 113.4491) (end 126.3142 113.4491) (width 0.5) (layer F.Cu) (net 42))
 (segment (start 115.12 108.372) (end 115.12 112.464) (width 0.5) (layer F.Cu) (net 42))
 (segment (start 115.12 112.464) (end 116.1051 113.4491) (width 0.5) (layer F.Cu) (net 42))
 (segment (start 113.4 108.372) (end 115.12 108.372) (width 0.5) (layer F.Cu) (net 42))
 (segment (start 113.4 108.372) (end 113.4 117.083) (width 0.5) (layer F.Cu) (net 42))
 (segment (start 113.4 117.083) (end 113.792 117.475) (width 0.25) (layer F.Cu) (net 42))
 (segment (start 106.807 102.108) (end 106.807 102.287) (width 0.25) (layer F.Cu) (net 42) (status 30))
 (segment (start 124.6124 114.7191) (end 124.6124 113.4491) (width 0.25) (layer F.Cu) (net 42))
 (segment (start 116.1051 113.4491) (end 116.1051 115.0891) (width 0.5) (layer F.Cu) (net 42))
 (segment (start 116.1051 115.0891) (end 116.84 115.824) (width 0.5) (layer F.Cu) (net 42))
 (segment (start 116.84 115.824) (end 123.5075 115.824) (width 0.5) (layer F.Cu) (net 42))
 (segment (start 123.5075 115.824) (end 124.6124 114.7191) (width 0.5) (layer F.Cu) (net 42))
 (segment (start 109.306999 104.607999) (end 109.306999 104.734999) (width 0.25) (layer F.Cu) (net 42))
 (segment (start 106.807 102.108) (end 109.306999 104.607999) (width 2) (layer F.Cu) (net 42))
 (segment (start 109.306999 104.734999) (end 110.744 106.172) (width 2) (layer F.Cu) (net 42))
 (segment (start 110.744 114.427) (end 113.792 117.475) (width 2) (layer F.Cu) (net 42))
 (segment (start 110.744 106.172) (end 110.744 114.427) (width 2) (layer F.Cu) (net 42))
 (segment (start 150.406999 119.213001) (end 150.406999 119.087001) (width 0.25) (layer B.Cu) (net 40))
 (segment (start 149.732 119.888) (end 150.406999 119.213001) (width 0.25) (layer B.Cu) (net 40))
 (segment (start 150.406999 119.087001) (end 152.4 117.094) (width 0.25) (layer B.Cu) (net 40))
 (segment (start 158.9056 117.094) (end 164.2872 111.7124) (width 0.25) (layer B.Cu) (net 40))
 (segment (start 152.4 117.094) (end 158.9056 117.094) (width 0.25) (layer B.Cu) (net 40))
 (segment (start 129.7178 113.4491) (end 129.7178 118.7958) (width 0.25) (layer F.Cu) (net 41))
 (segment (start 129.7178 118.7958) (end 130.81 119.888) (width 0.25) (layer F.Cu) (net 41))
 (segment (start 130.9878 119.7102) (end 130.81 119.888) (width 0.25) (layer F.Cu) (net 41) (status 30))
 (segment (start 130.81 119.888) (end 132.81 119.888) (width 0.25) (layer F.Cu) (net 41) (status 30))
 (segment (start 132.81 119.888) (end 142.24 119.888) (width 0.25) (layer F.Cu) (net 41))
 (segment (start 158.8516 118.364) (end 164.2872 112.9284) (width 0.25) (layer B.Cu) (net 39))
 (segment (start 152.301406 118.364) (end 158.8516 118.364) (width 0.25) (layer B.Cu) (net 39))
 (segment (start 151.732 118.933406) (end 152.301406 118.364) (width 0.25) (layer B.Cu) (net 39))
 (segment (start 151.732 119.888) (end 151.732 118.933406) (width 0.25) (layer B.Cu) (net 39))
 (segment (start 158.5436 119.888) (end 164.2872 114.1444) (width 0.25) (layer B.Cu) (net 38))
 (segment (start 153.732 119.888) (end 158.5436 119.888) (width 0.25) (layer B.Cu) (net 38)))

